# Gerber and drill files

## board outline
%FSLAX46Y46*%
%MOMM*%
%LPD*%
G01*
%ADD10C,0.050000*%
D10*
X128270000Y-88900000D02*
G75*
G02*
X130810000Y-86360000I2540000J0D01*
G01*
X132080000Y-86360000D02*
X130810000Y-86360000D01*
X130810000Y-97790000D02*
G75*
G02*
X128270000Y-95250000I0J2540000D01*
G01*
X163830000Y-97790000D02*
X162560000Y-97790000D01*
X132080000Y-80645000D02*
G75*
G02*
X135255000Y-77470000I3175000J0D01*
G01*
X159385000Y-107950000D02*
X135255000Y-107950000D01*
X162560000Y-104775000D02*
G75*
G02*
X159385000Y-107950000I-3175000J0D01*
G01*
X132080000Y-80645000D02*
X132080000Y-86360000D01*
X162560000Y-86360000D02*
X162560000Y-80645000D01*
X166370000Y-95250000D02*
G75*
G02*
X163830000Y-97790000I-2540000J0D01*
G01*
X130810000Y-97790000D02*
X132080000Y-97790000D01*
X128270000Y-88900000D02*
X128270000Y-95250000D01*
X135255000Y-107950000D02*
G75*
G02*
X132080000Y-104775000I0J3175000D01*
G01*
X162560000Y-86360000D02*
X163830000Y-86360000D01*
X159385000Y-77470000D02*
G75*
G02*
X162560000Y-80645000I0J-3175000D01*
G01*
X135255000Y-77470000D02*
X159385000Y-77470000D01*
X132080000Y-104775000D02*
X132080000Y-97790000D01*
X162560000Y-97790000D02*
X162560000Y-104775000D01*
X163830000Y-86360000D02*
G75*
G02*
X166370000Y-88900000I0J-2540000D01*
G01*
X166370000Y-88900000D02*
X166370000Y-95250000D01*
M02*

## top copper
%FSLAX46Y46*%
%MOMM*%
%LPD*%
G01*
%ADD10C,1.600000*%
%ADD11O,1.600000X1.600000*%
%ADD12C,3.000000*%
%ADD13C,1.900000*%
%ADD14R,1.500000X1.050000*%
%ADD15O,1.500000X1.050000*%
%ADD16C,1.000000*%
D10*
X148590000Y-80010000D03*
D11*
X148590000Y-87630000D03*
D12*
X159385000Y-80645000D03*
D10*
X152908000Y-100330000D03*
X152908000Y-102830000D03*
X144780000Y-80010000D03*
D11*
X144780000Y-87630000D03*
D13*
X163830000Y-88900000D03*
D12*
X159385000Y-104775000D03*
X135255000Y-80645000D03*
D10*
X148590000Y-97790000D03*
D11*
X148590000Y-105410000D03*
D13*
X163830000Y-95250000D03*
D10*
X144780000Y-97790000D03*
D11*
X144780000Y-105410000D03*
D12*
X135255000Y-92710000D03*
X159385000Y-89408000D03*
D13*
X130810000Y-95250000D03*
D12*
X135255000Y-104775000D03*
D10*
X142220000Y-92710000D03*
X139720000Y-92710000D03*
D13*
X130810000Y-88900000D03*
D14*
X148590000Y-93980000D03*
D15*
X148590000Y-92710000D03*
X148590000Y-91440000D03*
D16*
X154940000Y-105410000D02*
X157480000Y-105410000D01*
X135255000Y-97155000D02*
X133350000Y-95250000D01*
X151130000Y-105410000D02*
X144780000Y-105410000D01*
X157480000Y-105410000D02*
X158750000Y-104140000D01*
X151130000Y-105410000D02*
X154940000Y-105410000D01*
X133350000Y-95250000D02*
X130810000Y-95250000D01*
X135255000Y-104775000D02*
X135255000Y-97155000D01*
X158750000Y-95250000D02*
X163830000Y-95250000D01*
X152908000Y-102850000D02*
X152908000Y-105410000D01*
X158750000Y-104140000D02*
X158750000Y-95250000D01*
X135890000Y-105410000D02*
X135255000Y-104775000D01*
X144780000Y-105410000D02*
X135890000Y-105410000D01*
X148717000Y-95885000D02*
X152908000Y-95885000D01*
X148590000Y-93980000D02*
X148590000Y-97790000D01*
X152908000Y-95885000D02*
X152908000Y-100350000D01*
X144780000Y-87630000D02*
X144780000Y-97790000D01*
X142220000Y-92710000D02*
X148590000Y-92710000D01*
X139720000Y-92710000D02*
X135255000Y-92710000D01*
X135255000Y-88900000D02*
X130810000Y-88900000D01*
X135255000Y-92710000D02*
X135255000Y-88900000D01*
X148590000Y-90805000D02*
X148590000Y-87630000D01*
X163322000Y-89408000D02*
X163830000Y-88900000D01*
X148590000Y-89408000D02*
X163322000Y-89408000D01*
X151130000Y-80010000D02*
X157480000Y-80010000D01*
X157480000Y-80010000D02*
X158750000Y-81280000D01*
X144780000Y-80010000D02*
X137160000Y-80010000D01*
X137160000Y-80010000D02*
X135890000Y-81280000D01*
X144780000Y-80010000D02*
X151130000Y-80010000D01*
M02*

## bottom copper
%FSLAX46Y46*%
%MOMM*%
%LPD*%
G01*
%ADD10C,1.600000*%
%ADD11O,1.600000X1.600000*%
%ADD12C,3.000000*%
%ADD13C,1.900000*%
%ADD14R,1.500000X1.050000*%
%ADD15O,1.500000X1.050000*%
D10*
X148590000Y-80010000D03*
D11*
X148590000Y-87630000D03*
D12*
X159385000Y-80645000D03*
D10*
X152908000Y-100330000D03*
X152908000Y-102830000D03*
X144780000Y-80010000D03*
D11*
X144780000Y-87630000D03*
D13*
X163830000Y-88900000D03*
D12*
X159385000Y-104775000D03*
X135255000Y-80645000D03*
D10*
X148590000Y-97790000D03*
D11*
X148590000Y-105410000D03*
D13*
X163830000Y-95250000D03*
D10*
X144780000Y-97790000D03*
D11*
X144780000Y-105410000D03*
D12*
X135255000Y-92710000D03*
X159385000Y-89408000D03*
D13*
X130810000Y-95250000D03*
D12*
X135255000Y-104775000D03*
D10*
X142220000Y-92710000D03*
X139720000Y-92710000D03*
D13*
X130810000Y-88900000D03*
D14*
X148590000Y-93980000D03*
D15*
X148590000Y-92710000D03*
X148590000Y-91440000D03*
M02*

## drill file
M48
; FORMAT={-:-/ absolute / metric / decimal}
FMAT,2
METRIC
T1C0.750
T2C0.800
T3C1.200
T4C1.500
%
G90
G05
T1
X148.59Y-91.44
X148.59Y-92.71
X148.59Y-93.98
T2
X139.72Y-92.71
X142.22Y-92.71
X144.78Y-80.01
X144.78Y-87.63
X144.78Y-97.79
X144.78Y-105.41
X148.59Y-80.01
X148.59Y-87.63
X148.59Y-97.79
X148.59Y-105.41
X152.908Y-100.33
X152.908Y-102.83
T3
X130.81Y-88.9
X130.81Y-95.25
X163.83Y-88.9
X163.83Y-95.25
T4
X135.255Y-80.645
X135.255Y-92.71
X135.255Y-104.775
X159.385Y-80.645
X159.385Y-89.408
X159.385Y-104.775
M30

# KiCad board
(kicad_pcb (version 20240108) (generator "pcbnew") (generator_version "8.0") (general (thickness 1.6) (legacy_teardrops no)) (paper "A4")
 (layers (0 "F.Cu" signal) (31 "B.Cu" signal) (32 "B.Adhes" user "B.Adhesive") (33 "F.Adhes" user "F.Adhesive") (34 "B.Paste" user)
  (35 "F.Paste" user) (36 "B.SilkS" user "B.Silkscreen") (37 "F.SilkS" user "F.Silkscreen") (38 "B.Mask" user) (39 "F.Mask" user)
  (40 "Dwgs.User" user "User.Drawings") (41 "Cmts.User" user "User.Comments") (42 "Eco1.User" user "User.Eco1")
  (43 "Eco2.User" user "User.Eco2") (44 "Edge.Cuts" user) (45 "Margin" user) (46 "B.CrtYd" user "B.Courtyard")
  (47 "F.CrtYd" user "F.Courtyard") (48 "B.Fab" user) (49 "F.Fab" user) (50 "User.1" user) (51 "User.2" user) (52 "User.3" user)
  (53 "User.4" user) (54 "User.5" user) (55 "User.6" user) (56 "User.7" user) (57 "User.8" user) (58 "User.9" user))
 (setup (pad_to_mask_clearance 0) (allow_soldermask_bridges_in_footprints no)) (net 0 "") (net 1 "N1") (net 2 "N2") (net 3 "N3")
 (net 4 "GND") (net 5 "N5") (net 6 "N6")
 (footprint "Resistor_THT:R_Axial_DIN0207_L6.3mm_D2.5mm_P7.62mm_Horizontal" (layer "F.Cu") (at 148.59 80.01 -90)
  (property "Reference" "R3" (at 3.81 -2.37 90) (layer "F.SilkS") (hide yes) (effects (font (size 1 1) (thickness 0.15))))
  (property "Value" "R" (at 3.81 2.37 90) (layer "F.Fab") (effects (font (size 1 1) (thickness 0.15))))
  (pad "1" thru_hole circle (at 0 0 270) (size 1.6 1.6) (drill 0.8) (layers "*.Cu" "*.Mask") (remove_unused_layers no) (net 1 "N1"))
  (pad "2" thru_hole oval (at 7.62 0 270) (size 1.6 1.6) (drill 0.8) (layers "*.Cu" "*.Mask") (remove_unused_layers no) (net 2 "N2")))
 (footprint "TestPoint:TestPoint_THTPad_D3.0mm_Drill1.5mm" (layer "F.Cu") (at 159.385 80.645)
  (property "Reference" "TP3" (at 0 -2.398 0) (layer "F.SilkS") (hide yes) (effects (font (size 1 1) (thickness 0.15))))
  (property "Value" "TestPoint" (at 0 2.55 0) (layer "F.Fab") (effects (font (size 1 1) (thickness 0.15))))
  (pad "1" thru_hole circle (at 0 0) (size 3 3) (drill 1.5) (layers "*.Cu" "*.Mask") (remove_unused_layers no) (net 1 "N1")))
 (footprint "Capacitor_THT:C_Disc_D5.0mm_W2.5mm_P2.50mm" (layer "F.Cu") (at 152.908 100.33 -90)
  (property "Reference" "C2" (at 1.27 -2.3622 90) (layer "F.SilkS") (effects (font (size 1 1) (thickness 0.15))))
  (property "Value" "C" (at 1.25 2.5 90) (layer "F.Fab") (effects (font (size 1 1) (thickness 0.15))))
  (pad "1" thru_hole circle (at 0 0 270) (size 1.6 1.6) (drill 0.8) (layers "*.Cu" "*.Mask") (remove_unused_layers no) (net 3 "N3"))
  (pad "2" thru_hole circle (at 2.5 0 270) (size 1.6 1.6) (drill 0.8) (layers "*.Cu" "*.Mask") (remove_unused_layers no) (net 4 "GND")))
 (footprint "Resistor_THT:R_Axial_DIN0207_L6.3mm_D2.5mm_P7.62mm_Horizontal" (layer "F.Cu") (at 144.78 80.01 -90)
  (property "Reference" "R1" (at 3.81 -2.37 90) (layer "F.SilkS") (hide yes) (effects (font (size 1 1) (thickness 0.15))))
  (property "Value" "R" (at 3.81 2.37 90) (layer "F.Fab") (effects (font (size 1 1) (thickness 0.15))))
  (pad "1" thru_hole circle (at 0 0 270) (size 1.6 1.6) (drill 0.8) (layers "*.Cu" "*.Mask") (remove_unused_layers no) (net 1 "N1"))
  (pad "2" thru_hole oval (at 7.62 0 270) (size 1.6 1.6) (drill 0.8) (layers "*.Cu" "*.Mask") (remove_unused_layers no) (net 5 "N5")))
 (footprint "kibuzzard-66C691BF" (layer "F.Cu") (at 159.385 96.774 90)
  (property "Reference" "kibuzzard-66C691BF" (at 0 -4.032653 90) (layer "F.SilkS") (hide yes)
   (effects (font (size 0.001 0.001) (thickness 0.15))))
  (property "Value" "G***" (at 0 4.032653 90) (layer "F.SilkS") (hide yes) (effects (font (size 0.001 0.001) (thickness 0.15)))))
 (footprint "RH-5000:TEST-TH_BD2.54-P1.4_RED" (layer "F.Cu") (at 163.83 88.9)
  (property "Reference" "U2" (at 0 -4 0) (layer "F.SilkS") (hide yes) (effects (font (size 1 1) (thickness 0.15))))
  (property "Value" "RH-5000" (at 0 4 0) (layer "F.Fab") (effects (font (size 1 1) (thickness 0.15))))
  (pad "1" thru_hole circle (at 0 0) (size 1.9 1.9) (drill 1.199998) (layers "*.Cu" "*.Paste" "*.Mask") (remove_unused_layers no)
   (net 2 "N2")))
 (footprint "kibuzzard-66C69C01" (layer "F.Cu") (at 153.67 83.82 90)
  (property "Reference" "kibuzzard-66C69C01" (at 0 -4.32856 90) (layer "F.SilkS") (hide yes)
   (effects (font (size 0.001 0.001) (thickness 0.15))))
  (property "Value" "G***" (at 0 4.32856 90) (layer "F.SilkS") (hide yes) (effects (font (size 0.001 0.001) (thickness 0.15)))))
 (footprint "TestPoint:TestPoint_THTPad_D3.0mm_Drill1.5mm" (layer "F.Cu") (at 159.385 104.775)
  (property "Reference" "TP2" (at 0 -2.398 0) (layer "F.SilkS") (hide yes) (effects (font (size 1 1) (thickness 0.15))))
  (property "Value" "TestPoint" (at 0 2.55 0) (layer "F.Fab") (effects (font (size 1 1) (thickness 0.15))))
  (pad "1" thru_hole circle (at 0 0) (size 3 3) (drill 1.5) (layers "*.Cu" "*.Mask") (remove_unused_layers no) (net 4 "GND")))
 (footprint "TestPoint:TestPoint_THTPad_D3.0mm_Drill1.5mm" (layer "F.Cu") (at 135.255 80.645)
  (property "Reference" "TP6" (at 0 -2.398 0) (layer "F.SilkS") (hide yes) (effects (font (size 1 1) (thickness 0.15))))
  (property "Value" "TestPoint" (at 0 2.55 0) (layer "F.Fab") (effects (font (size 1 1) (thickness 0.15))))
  (pad "1" thru_hole circle (at 0 0) (size 3 3) (drill 1.5) (layers "*.Cu" "*.Mask") (remove_unused_layers no) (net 1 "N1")))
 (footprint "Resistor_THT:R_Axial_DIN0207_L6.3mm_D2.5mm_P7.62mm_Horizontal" (layer "F.Cu") (at 148.59 97.79 -90)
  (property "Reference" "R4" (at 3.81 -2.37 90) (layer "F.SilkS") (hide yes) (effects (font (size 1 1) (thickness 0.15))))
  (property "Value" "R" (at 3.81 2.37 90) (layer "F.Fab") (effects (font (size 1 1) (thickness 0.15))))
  (pad "1" thru_hole circle (at 0 0 270) (size 1.6 1.6) (drill 0.8) (layers "*.Cu" "*.Mask") (remove_unused_layers no) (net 3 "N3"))
  (pad "2" thru_hole oval (at 7.62 0 270) (size 1.6 1.6) (drill 0.8) (layers "*.Cu" "*.Mask") (remove_unused_layers no) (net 4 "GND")))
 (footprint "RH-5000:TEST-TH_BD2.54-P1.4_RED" (layer "F.Cu") (at 163.83 95.25)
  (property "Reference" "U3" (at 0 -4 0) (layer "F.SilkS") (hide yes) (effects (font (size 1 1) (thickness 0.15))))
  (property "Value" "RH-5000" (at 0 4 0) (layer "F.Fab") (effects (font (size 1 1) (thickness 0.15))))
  (pad "1" thru_hole circle (at 0 0) (size 1.9 1.9) (drill 1.199998) (layers "*.Cu" "*.Paste" "*.Mask") (remove_unused_layers no)
   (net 4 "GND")))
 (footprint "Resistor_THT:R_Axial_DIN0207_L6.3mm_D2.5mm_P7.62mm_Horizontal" (layer "F.Cu") (at 144.78 97.79 -90)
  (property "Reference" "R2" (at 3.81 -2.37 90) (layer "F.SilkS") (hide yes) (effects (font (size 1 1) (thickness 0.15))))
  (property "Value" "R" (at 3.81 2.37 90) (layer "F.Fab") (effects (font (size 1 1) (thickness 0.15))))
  (pad "1" thru_hole circle (at 0 0 270) (size 1.6 1.6) (drill 0.8) (layers "*.Cu" "*.Mask") (remove_unused_layers no) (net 5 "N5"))
  (pad "2" thru_hole oval (at 7.62 0 270) (size 1.6 1.6) (drill 0.8) (layers "*.Cu" "*.Mask") (remove_unused_layers no) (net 4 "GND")))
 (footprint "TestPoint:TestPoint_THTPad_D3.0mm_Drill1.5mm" (layer "F.Cu") (at 135.255 92.71)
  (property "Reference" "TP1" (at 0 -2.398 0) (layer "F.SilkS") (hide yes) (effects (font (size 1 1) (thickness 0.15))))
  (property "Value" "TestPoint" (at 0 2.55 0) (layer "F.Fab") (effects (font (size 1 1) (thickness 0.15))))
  (pad "1" thru_hole circle (at 0 0) (size 3 3) (drill 1.5) (layers "*.Cu" "*.Mask") (remove_unused_layers no) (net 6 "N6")))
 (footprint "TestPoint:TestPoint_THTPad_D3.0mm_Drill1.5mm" (layer "F.Cu") (at 159.385 89.408)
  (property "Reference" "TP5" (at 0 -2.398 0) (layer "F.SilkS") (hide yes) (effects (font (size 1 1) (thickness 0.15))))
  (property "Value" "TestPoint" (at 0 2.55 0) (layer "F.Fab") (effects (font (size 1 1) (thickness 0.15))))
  (pad "1" thru_hole circle (at 0 0) (size 3 3) (drill 1.5) (layers "*.Cu" "*.Mask") (remove_unused_layers no) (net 2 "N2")))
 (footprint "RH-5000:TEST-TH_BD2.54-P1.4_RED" (layer "F.Cu") (at 130.81 95.25)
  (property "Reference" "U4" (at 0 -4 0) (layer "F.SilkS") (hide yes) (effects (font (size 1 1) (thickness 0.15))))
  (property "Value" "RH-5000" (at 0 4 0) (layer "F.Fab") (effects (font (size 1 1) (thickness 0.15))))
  (pad "1" thru_hole circle (at 0 0) (size 1.9 1.9) (drill 1.199998) (layers "*.Cu" "*.Paste" "*.Mask") (remove_unused_layers no)
   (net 4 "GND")))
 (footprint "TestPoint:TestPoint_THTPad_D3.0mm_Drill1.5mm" (layer "F.Cu") (at 135.255 104.775)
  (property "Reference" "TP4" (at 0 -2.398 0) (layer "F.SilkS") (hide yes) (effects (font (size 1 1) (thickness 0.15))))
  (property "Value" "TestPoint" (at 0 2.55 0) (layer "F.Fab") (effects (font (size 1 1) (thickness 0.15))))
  (pad "1" thru_hole circle (at 0 0) (size 3 3) (drill 1.5) (layers "*.Cu" "*.Mask") (remove_unused_layers no) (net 4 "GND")))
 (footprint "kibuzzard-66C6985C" (layer "F.Cu") (at 135.89 98.298 90)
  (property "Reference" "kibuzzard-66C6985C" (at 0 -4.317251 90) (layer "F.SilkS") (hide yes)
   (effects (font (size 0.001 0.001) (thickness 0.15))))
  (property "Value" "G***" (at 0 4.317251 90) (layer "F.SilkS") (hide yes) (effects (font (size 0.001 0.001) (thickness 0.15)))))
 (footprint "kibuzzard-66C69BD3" (layer "F.Cu") (at 135.89 86.868 90)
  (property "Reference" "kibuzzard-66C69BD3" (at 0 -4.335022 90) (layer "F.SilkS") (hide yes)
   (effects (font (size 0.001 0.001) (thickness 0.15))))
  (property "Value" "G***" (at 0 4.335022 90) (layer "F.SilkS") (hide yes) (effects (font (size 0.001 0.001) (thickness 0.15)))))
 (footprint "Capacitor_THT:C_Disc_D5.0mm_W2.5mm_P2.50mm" (layer "F.Cu") (at 142.22 92.71 180)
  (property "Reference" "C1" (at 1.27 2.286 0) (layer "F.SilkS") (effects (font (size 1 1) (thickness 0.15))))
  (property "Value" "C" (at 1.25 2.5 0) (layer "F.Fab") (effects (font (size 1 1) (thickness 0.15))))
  (pad "1" thru_hole circle (at 0 0 180) (size 1.6 1.6) (drill 0.8) (layers "*.Cu" "*.Mask") (remove_unused_layers no) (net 5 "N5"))
  (pad "2" thru_hole circle (at 2.5 0 180) (size 1.6 1.6) (drill 0.8) (layers "*.Cu" "*.Mask") (remove_unused_layers no) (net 6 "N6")))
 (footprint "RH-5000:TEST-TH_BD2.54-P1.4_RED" (layer "F.Cu") (at 130.81 88.9)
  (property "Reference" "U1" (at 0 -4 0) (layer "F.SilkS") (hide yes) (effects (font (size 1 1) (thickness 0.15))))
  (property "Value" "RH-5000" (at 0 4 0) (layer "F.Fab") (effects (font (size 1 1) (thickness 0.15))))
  (pad "1" thru_hole circle (at 0 0) (size 1.9 1.9) (drill 1.199998) (layers "*.Cu" "*.Paste" "*.Mask") (remove_unused_layers no)
   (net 6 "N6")))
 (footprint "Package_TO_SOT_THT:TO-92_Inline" (layer "F.Cu") (at 148.59 93.98 90)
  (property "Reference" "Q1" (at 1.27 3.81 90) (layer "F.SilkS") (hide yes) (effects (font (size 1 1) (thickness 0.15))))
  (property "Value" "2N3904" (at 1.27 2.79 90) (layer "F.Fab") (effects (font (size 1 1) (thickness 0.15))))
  (pad "1" thru_hole rect (at 0 0 90) (size 1.05 1.5) (drill 0.75) (layers "*.Cu" "*.Mask") (remove_unused_layers no) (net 3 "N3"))
  (pad "2" thru_hole oval (at 1.27 0 90) (size 1.05 1.5) (drill 0.75) (layers "*.Cu" "*.Mask") (remove_unused_layers no) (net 5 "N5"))
  (pad "3" thru_hole oval (at 2.54 0 90) (size 1.05 1.5) (drill 0.75) (layers "*.Cu" "*.Mask") (remove_unused_layers no) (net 2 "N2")))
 (gr_arc (start 128.27 88.9) (mid 129.013949 87.103949) (end 130.81 86.36) (stroke (width 0.05) (type default)) (layer "Edge.Cuts"))
 (gr_line (start 132.08 86.36) (end 130.81 86.36) (stroke (width 0.05) (type default)) (layer "Edge.Cuts"))
 (gr_arc (start 130.81 97.79) (mid 129.013949 97.046051) (end 128.27 95.25) (stroke (width 0.05) (type default)) (layer "Edge.Cuts"))
 (gr_line (start 163.83 97.79) (end 162.56 97.79) (stroke (width 0.05) (type default)) (layer "Edge.Cuts"))
 (gr_arc (start 132.08 80.645) (mid 133.009936 78.399936) (end 135.255 77.47) (stroke (width 0.05) (type default)) (layer "Edge.Cuts"))
 (gr_line (start 159.385 107.95) (end 135.255 107.95) (stroke (width 0.05) (type default)) (layer "Edge.Cuts"))
 (gr_arc (start 162.56 104.775) (mid 161.630064 107.020064) (end 159.385 107.95) (stroke (width 0.05) (type default)) (layer "Edge.Cuts"))
 (gr_line (start 132.08 80.645) (end 132.08 86.36) (stroke (width 0.05) (type default)) (layer "Edge.Cuts"))
 (gr_line (start 162.56 86.36) (end 162.56 80.645) (stroke (width 0.05) (type default)) (layer "Edge.Cuts"))
 (gr_arc (start 166.37 95.25) (mid 165.626051 97.046051) (end 163.83 97.79) (stroke (width 0.05) (type default)) (layer "Edge.Cuts"))
 (gr_line (start 130.81 97.79) (end 132.08 97.79) (stroke (width 0.05) (type default)) (layer "Edge.Cuts"))
 (gr_line (start 128.27 88.9) (end 128.27 95.25) (stroke (width 0.05) (type default)) (layer "Edge.Cuts"))
 (gr_arc (start 135.255 107.95) (mid 133.009936 107.020064) (end 132.08 104.775) (stroke (width 0.05) (type default)) (layer "Edge.Cuts"))
 (gr_line (start 162.56 86.36) (end 163.83 86.36) (stroke (width 0.05) (type default)) (layer "Edge.Cuts"))
 (gr_arc (start 159.385 77.47) (mid 161.630064 78.399936) (end 162.56 80.645) (stroke (width 0.05) (type default)) (layer "Edge.Cuts"))
 (gr_line (start 135.255 77.47) (end 159.385 77.47) (stroke (width 0.05) (type default)) (layer "Edge.Cuts"))
 (gr_line (start 132.08 104.775) (end 132.08 97.79) (stroke (width 0.05) (type default)) (layer "Edge.Cuts"))
 (gr_line (start 162.56 97.79) (end 162.56 104.775) (stroke (width 0.05) (type default)) (layer "Edge.Cuts"))
 (gr_arc (start 163.83 86.36) (mid 165.626051 87.103949) (end 166.37 88.9) (stroke (width 0.05) (type default)) (layer "Edge.Cuts"))
 (gr_line (start 166.37 88.9) (end 166.37 95.25) (stroke (width 0.05) (type default)) (layer "Edge.Cuts"))
 (segment (start 154.94 105.41) (end 157.48 105.41) (width 1) (layer "F.Cu") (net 4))
 (segment (start 135.255 97.155) (end 133.35 95.25) (width 1) (layer "F.Cu") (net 4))
 (segment (start 151.13 105.41) (end 144.78 105.41) (width 1) (layer "F.Cu") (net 4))
 (segment (start 157.48 105.41) (end 158.75 104.14) (width 1) (layer "F.Cu") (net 4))
 (segment (start 151.13 105.41) (end 154.94 105.41) (width 1) (layer "F.Cu") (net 4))
 (segment (start 133.35 95.25) (end 130.81 95.25) (width 1) (layer "F.Cu") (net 4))
 (segment (start 135.255 104.775) (end 135.255 97.155) (width 1) (layer "F.Cu") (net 4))
 (segment (start 158.75 95.25) (end 163.83 95.25) (width 1) (layer "F.Cu") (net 4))
 (segment (start 152.908 102.85) (end 152.908 105.41) (width 1) (layer "F.Cu") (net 4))
 (segment (start 158.75 104.14) (end 158.75 95.25) (width 1) (layer "F.Cu") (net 4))
 (segment (start 135.89 105.41) (end 135.255 104.775) (width 1) (layer "F.Cu") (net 4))
 (segment (start 144.78 105.41) (end 135.89 105.41) (width 1) (layer "F.Cu") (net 4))
 (segment (start 148.717 95.885) (end 152.908 95.885) (width 1) (layer "F.Cu") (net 3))
 (segment (start 148.59 93.98) (end 148.59 97.79) (width 1) (layer "F.Cu") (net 3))
 (segment (start 152.908 95.885) (end 152.908 100.35) (width 1) (layer "F.Cu") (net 3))
 (segment (start 144.78 87.63) (end 144.78 97.79) (width 1) (layer "F.Cu") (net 5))
 (segment (start 142.22 92.71) (end 148.59 92.71) (width 1) (layer "F.Cu") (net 5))
 (segment (start 139.72 92.71) (end 135.255 92.71) (width 1) (layer "F.Cu") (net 6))
 (segment (start 135.255 88.9) (end 130.81 88.9) (width 1) (layer "F.Cu") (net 6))
 (segment (start 135.255 92.71) (end 135.255 88.9) (width 1) (layer "F.Cu") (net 6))
 (segment (start 148.59 90.805) (end 148.59 87.63) (width 1) (layer "F.Cu") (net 2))
 (segment (start 163.322 89.408) (end 163.83 88.9) (width 1) (layer "F.Cu") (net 2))
 (segment (start 148.59 89.408) (end 163.322 89.408) (width 1) (layer "F.Cu") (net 2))
 (segment (start 151.13 80.01) (end 157.48 80.01) (width 1) (layer "F.Cu") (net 1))
 (segment (start 157.48 80.01) (end 158.75 81.28) (width 1) (layer "F.Cu") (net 1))
 (segment (start 144.78 80.01) (end 137.16 80.01) (width 1) (layer "F.Cu") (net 1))
 (segment (start 137.16 80.01) (end 135.89 81.28) (width 1) (layer "F.Cu") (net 1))
 (segment (start 144.78 80.01) (end 151.13 80.01) (width 1) (layer "F.Cu") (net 1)))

